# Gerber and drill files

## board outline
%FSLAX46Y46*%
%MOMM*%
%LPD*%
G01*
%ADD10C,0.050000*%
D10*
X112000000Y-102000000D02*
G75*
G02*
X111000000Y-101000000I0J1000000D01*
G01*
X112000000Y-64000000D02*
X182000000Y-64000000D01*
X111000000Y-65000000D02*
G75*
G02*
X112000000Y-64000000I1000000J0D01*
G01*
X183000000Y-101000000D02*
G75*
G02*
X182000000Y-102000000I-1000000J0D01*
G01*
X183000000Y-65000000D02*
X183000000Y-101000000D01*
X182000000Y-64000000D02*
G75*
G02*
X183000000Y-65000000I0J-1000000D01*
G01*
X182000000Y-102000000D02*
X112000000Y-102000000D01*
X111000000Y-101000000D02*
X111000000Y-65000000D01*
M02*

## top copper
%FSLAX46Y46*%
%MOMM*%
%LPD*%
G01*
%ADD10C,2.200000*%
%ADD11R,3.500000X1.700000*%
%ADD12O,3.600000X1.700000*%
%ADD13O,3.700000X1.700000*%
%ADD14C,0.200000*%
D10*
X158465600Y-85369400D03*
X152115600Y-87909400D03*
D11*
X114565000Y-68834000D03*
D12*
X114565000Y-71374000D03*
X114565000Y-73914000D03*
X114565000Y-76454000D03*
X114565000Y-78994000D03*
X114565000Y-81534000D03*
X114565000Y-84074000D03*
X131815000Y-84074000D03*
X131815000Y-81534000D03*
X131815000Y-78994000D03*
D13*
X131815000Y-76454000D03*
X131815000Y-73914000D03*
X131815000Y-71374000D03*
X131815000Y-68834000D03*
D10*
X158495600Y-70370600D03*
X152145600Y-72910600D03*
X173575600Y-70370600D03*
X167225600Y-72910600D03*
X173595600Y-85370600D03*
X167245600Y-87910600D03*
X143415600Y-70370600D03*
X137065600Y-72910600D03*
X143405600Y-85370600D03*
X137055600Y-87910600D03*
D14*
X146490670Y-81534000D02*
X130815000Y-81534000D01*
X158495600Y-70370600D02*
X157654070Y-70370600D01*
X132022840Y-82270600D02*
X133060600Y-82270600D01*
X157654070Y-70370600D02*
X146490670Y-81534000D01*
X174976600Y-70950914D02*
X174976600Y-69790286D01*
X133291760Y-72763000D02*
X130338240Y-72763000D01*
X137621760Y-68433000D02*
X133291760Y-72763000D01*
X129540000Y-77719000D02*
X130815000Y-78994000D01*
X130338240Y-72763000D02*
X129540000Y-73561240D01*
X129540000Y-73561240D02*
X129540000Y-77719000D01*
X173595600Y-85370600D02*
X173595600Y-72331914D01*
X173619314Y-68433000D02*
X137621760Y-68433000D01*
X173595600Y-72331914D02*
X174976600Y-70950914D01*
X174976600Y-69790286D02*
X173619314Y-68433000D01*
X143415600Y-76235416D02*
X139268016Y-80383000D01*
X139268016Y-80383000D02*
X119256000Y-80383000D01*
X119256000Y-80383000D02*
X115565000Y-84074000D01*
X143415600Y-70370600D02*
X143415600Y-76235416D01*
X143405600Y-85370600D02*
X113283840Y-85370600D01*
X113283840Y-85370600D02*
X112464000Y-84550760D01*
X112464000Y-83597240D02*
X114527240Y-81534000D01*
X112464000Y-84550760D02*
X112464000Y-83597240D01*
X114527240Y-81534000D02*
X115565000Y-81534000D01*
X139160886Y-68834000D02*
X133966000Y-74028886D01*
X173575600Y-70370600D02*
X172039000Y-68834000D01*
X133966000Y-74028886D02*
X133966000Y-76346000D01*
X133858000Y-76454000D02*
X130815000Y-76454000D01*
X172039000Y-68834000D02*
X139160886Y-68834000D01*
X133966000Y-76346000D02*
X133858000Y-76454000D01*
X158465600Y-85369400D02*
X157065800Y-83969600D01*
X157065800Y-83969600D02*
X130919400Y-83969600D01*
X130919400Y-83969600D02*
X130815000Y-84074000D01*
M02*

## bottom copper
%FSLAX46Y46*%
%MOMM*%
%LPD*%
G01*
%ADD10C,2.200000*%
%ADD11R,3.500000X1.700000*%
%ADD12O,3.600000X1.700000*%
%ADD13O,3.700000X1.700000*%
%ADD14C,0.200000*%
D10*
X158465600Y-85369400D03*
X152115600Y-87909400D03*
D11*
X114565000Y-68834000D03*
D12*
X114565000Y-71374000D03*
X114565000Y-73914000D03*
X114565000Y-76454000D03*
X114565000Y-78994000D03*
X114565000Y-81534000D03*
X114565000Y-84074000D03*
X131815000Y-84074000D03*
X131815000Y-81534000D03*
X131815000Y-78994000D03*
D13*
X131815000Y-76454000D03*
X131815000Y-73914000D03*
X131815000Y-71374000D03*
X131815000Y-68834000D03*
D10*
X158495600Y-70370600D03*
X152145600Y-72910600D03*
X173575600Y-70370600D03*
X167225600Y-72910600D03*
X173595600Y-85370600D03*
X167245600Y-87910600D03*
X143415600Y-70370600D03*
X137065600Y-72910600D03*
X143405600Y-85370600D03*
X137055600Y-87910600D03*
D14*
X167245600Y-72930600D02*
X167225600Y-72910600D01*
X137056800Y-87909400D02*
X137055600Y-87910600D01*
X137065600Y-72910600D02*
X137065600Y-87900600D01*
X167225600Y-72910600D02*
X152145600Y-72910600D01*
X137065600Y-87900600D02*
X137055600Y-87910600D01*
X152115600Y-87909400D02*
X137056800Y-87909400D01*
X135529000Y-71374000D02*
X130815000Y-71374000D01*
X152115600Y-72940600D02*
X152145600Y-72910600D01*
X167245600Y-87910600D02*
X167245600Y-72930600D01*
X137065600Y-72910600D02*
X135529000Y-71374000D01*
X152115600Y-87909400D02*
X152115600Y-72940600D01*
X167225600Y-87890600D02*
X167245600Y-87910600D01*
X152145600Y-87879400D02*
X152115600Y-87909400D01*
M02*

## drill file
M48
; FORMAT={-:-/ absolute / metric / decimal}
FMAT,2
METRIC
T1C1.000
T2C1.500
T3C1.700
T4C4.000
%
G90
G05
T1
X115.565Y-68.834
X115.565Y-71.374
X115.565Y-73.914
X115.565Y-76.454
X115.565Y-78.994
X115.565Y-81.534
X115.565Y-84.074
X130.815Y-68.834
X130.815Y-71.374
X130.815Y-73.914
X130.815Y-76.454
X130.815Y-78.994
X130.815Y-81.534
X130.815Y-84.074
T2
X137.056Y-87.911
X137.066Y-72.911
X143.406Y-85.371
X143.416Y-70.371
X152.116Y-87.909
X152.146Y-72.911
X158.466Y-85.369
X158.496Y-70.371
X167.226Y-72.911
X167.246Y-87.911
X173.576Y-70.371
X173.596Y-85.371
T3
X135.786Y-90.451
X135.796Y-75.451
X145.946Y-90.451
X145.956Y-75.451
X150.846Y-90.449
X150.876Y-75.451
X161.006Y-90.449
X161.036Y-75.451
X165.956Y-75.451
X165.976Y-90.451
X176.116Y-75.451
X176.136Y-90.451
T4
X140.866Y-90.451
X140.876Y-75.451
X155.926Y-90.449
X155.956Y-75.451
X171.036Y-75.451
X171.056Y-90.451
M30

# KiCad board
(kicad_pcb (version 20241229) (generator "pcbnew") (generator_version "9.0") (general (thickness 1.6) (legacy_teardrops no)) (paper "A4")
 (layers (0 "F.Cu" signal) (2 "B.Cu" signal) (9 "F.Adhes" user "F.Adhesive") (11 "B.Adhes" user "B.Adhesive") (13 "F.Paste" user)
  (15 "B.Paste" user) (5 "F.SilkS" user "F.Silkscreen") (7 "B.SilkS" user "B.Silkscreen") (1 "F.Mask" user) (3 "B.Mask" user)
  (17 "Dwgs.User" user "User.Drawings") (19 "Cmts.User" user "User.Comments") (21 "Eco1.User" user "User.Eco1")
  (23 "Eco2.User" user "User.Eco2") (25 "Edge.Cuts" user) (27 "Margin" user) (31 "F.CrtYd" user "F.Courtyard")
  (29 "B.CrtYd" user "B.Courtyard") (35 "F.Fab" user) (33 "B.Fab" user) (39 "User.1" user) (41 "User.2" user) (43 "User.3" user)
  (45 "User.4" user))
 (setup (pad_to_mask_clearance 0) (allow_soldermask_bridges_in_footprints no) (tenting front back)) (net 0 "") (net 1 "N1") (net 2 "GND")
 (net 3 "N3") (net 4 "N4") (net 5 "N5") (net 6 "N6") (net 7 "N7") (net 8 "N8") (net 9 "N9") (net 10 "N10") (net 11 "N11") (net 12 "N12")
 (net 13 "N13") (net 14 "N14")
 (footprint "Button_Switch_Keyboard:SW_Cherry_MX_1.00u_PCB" (layer "F.Cu") (at 158.4656 85.3694)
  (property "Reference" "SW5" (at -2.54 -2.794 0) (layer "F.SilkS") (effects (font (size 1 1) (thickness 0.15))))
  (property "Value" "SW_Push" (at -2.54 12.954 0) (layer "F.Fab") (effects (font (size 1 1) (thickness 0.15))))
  (pad "" np_thru_hole circle (at -7.62 5.08) (size 1.7 1.7) (drill 1.7) (layers "*.Cu" "*.Mask"))
  (pad "" np_thru_hole circle (at -2.54 5.08) (size 4 4) (drill 4) (layers "*.Cu" "*.Mask"))
  (pad "" np_thru_hole circle (at 2.54 5.08) (size 1.7 1.7) (drill 1.7) (layers "*.Cu" "*.Mask"))
  (pad "1" thru_hole circle (at 0 0) (size 2.2 2.2) (drill 1.5) (layers "*.Cu" "*.Mask") (remove_unused_layers no) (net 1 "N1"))
  (pad "2" thru_hole circle (at -6.35 2.54) (size 2.2 2.2) (drill 1.5) (layers "*.Cu" "*.Mask") (remove_unused_layers no) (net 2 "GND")))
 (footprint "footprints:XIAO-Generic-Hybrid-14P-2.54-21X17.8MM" (layer "F.Cu") (at 123.19 76.454)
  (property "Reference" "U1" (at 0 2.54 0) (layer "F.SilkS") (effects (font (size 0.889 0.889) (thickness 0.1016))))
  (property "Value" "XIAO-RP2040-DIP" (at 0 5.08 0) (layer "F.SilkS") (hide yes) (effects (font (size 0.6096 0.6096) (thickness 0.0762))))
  (pad "1" thru_hole rect (at -7.625 -7.62) (size 3.5 1.7) (drill 1 (offset -1 0)) (layers "*.Cu" "*.Mask") (remove_unused_layers no)
   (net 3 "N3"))
  (pad "2" thru_hole oval (at -7.625 -5.08) (size 3.6 1.7) (drill 1 (offset -1 0)) (layers "*.Cu" "*.Mask") (remove_unused_layers no)
   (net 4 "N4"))
  (pad "3" thru_hole oval (at -7.625 -2.54) (size 3.6 1.7) (drill 1 (offset -1 0)) (layers "*.Cu" "*.Mask") (remove_unused_layers no)
   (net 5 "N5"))
  (pad "4" thru_hole oval (at -7.625 0) (size 3.6 1.7) (drill 1 (offset -1 0)) (layers "*.Cu" "*.Mask") (remove_unused_layers no)
   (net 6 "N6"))
  (pad "5" thru_hole oval (at -7.625 2.54) (size 3.6 1.7) (drill 1 (offset -1 0)) (layers "*.Cu" "*.Mask") (remove_unused_layers no)
   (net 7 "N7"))
  (pad "6" thru_hole oval (at -7.625 5.08 180) (size 3.6 1.7) (drill 1 (offset 1 0)) (layers "*.Cu" "*.Mask") (remove_unused_layers no)
   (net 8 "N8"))
  (pad "7" thru_hole oval (at -7.625 7.62) (size 3.6 1.7) (drill 1 (offset -1 0)) (layers "*.Cu" "*.Mask") (remove_unused_layers no)
   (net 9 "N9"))
  (pad "8" thru_hole oval (at 7.625 7.62) (size 3.6 1.7) (drill 1 (offset 1 0)) (layers "*.Cu" "*.Mask") (remove_unused_layers no)
   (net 1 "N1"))
  (pad "9" thru_hole oval (at 7.625 5.08) (size 3.6 1.7) (drill 1 (offset 1 0)) (layers "*.Cu" "*.Mask") (remove_unused_layers no)
   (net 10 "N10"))
  (pad "10" thru_hole oval (at 7.625 2.54) (size 3.6 1.7) (drill 1 (offset 1 0)) (layers "*.Cu" "*.Mask") (remove_unused_layers no)
   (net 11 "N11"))
  (pad "11" thru_hole oval (at 7.625 0) (size 3.7 1.7) (drill 1 (offset 1 0)) (layers "*.Cu" "*.Mask") (remove_unused_layers no)
   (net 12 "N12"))
  (pad "12" thru_hole oval (at 7.625 -2.54) (size 3.7 1.7) (drill 1 (offset 1 0)) (layers "*.Cu" "*.Mask") (remove_unused_layers no)
   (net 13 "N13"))
  (pad "13" thru_hole oval (at 7.625 -5.08) (size 3.7 1.7) (drill 1 (offset 1 0)) (layers "*.Cu" "*.Mask") (remove_unused_layers no)
   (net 2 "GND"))
  (pad "14" thru_hole oval (at 7.625 -7.62) (size 3.7 1.7) (drill 1 (offset 1 0)) (layers "*.Cu" "*.Mask") (remove_unused_layers no)
   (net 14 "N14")))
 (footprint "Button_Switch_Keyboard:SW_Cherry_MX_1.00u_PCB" (layer "F.Cu") (at 158.4956 70.3706)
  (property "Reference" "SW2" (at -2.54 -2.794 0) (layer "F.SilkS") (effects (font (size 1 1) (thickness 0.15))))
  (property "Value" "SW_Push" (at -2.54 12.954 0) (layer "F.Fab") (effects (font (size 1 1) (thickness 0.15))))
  (pad "" np_thru_hole circle (at -7.62 5.08) (size 1.7 1.7) (drill 1.7) (layers "*.Cu" "*.Mask"))
  (pad "" np_thru_hole circle (at -2.54 5.08) (size 4 4) (drill 4) (layers "*.Cu" "*.Mask"))
  (pad "" np_thru_hole circle (at 2.54 5.08) (size 1.7 1.7) (drill 1.7) (layers "*.Cu" "*.Mask"))
  (pad "1" thru_hole circle (at 0 0) (size 2.2 2.2) (drill 1.5) (layers "*.Cu" "*.Mask") (remove_unused_layers no) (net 10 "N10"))
  (pad "2" thru_hole circle (at -6.35 2.54) (size 2.2 2.2) (drill 1.5) (layers "*.Cu" "*.Mask") (remove_unused_layers no) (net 2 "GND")))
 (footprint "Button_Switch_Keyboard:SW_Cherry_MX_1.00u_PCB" (layer "F.Cu") (at 173.5756 70.3706)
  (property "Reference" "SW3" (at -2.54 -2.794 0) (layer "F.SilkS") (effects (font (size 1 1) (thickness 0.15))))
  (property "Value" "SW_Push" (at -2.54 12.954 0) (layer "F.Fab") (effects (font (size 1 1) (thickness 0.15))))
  (pad "" np_thru_hole circle (at -7.62 5.08) (size 1.7 1.7) (drill 1.7) (layers "*.Cu" "*.Mask"))
  (pad "" np_thru_hole circle (at -2.54 5.08) (size 4 4) (drill 4) (layers "*.Cu" "*.Mask"))
  (pad "" np_thru_hole circle (at 2.54 5.08) (size 1.7 1.7) (drill 1.7) (layers "*.Cu" "*.Mask"))
  (pad "1" thru_hole circle (at 0 0) (size 2.2 2.2) (drill 1.5) (layers "*.Cu" "*.Mask") (remove_unused_layers no) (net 12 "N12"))
  (pad "2" thru_hole circle (at -6.35 2.54) (size 2.2 2.2) (drill 1.5) (layers "*.Cu" "*.Mask") (remove_unused_layers no) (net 2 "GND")))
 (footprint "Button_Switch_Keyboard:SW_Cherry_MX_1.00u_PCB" (layer "F.Cu") (at 173.5956 85.3706)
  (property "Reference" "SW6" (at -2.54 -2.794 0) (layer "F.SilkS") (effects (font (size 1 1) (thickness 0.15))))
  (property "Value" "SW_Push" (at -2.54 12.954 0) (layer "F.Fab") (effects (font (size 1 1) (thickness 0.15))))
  (pad "" np_thru_hole circle (at -7.62 5.08) (size 1.7 1.7) (drill 1.7) (layers "*.Cu" "*.Mask"))
  (pad "" np_thru_hole circle (at -2.54 5.08) (size 4 4) (drill 4) (layers "*.Cu" "*.Mask"))
  (pad "" np_thru_hole circle (at 2.54 5.08) (size 1.7 1.7) (drill 1.7) (layers "*.Cu" "*.Mask"))
  (pad "1" thru_hole circle (at 0 0) (size 2.2 2.2) (drill 1.5) (layers "*.Cu" "*.Mask") (remove_unused_layers no) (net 11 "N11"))
  (pad "2" thru_hole circle (at -6.35 2.54) (size 2.2 2.2) (drill 1.5) (layers "*.Cu" "*.Mask") (remove_unused_layers no) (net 2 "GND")))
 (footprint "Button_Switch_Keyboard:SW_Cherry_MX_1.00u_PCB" (layer "F.Cu") (at 143.4156 70.3706)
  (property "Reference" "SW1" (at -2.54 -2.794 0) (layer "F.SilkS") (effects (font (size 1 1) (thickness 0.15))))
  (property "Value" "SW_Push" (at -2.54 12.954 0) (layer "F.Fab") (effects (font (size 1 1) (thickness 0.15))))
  (pad "" np_thru_hole circle (at -7.62 5.08) (size 1.7 1.7) (drill 1.7) (layers "*.Cu" "*.Mask"))
  (pad "" np_thru_hole circle (at -2.54 5.08) (size 4 4) (drill 4) (layers "*.Cu" "*.Mask"))
  (pad "" np_thru_hole circle (at 2.54 5.08) (size 1.7 1.7) (drill 1.7) (layers "*.Cu" "*.Mask"))
  (pad "1" thru_hole circle (at 0 0) (size 2.2 2.2) (drill 1.5) (layers "*.Cu" "*.Mask") (remove_unused_layers no) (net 9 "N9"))
  (pad "2" thru_hole circle (at -6.35 2.54) (size 2.2 2.2) (drill 1.5) (layers "*.Cu" "*.Mask") (remove_unused_layers no) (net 2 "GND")))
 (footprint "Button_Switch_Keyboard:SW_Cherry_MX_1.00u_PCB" (layer "F.Cu") (at 143.4056 85.3706)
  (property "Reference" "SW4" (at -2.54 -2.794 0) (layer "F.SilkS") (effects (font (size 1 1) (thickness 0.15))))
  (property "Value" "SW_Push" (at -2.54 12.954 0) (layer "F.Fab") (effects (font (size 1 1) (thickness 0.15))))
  (pad "" np_thru_hole circle (at -7.62 5.08) (size 1.7 1.7) (drill 1.7) (layers "*.Cu" "*.Mask"))
  (pad "" np_thru_hole circle (at -2.54 5.08) (size 4 4) (drill 4) (layers "*.Cu" "*.Mask"))
  (pad "" np_thru_hole circle (at 2.54 5.08) (size 1.7 1.7) (drill 1.7) (layers "*.Cu" "*.Mask"))
  (pad "1" thru_hole circle (at 0 0) (size 2.2 2.2) (drill 1.5) (layers "*.Cu" "*.Mask") (remove_unused_layers no) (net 8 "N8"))
  (pad "2" thru_hole circle (at -6.35 2.54) (size 2.2 2.2) (drill 1.5) (layers "*.Cu" "*.Mask") (remove_unused_layers no) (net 2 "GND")))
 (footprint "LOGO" (layer "F.Cu") (at 123 94)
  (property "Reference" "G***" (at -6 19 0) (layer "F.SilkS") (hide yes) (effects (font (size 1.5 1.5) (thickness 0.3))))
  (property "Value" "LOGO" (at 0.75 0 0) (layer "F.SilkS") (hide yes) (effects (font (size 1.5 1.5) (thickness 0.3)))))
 (gr_arc (start 112 102) (mid 111.292893 101.707107) (end 111 101) (stroke (width 0.05) (type default)) (layer "Edge.Cuts"))
 (gr_line (start 112 64) (end 182 64) (stroke (width 0.05) (type default)) (layer "Edge.Cuts"))
 (gr_arc (start 111 65) (mid 111.292893 64.292893) (end 112 64) (stroke (width 0.05) (type default)) (layer "Edge.Cuts"))
 (gr_arc (start 183 101) (mid 182.707107 101.707107) (end 182 102) (stroke (width 0.05) (type default)) (layer "Edge.Cuts"))
 (gr_line (start 183 65) (end 183 101) (stroke (width 0.05) (type default)) (layer "Edge.Cuts"))
 (gr_arc (start 182 64) (mid 182.707107 64.292893) (end 183 65) (stroke (width 0.05) (type default)) (layer "Edge.Cuts"))
 (gr_line (start 182 102) (end 112 102) (stroke (width 0.05) (type default)) (layer "Edge.Cuts"))
 (gr_line (start 111 101) (end 111 65) (stroke (width 0.05) (type default)) (layer "Edge.Cuts"))
 (segment (start 146.49067 81.534) (end 130.815 81.534) (width 0.2) (layer "F.Cu") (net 10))
 (segment (start 158.4956 70.3706) (end 157.65407 70.3706) (width 0.2) (layer "F.Cu") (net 10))
 (segment (start 132.02284 82.2706) (end 133.0606 82.2706) (width 0.2) (layer "F.Cu") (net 10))
 (segment (start 157.65407 70.3706) (end 146.49067 81.534) (width 0.2) (layer "F.Cu") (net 10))
 (segment (start 167.2456 72.9306) (end 167.2256 72.9106) (width 0.2) (layer "B.Cu") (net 2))
 (segment (start 137.0568 87.9094) (end 137.0556 87.9106) (width 0.2) (layer "B.Cu") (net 2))
 (segment (start 137.0656 72.9106) (end 137.0656 87.9006) (width 0.2) (layer "B.Cu") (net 2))
 (segment (start 167.2256 72.9106) (end 152.1456 72.9106) (width 0.2) (layer "B.Cu") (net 2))
 (segment (start 137.0656 87.9006) (end 137.0556 87.9106) (width 0.2) (layer "B.Cu") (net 2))
 (segment (start 152.1156 87.9094) (end 137.0568 87.9094) (width 0.2) (layer "B.Cu") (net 2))
 (segment (start 135.529 71.374) (end 130.815 71.374) (width 0.2) (layer "B.Cu") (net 2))
 (segment (start 152.1156 72.9406) (end 152.1456 72.9106) (width 0.2) (layer "B.Cu") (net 2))
 (segment (start 167.2456 87.9106) (end 167.2456 72.9306) (width 0.2) (layer "B.Cu") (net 2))
 (segment (start 137.0656 72.9106) (end 135.529 71.374) (width 0.2) (layer "B.Cu") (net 2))
 (segment (start 152.1156 87.9094) (end 152.1156 72.9406) (width 0.2) (layer "B.Cu") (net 2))
 (segment (start 167.2256 87.8906) (end 167.2456 87.9106) (width 0.2) (layer "B.Cu") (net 2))
 (segment (start 152.1456 87.8794) (end 152.1156 87.9094) (width 0.2) (layer "B.Cu") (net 2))
 (segment (start 174.9766 70.950914) (end 174.9766 69.790286) (width 0.2) (layer "F.Cu") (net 11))
 (segment (start 133.29176 72.763) (end 130.33824 72.763) (width 0.2) (layer "F.Cu") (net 11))
 (segment (start 137.62176 68.433) (end 133.29176 72.763) (width 0.2) (layer "F.Cu") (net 11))
 (segment (start 129.54 77.719) (end 130.815 78.994) (width 0.2) (layer "F.Cu") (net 11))
 (segment (start 130.33824 72.763) (end 129.54 73.56124) (width 0.2) (layer "F.Cu") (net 11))
 (segment (start 129.54 73.56124) (end 129.54 77.719) (width 0.2) (layer "F.Cu") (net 11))
 (segment (start 173.5956 85.3706) (end 173.5956 72.331914) (width 0.2) (layer "F.Cu") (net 11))
 (segment (start 173.619314 68.433) (end 137.62176 68.433) (width 0.2) (layer "F.Cu") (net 11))
 (segment (start 173.5956 72.331914) (end 174.9766 70.950914) (width 0.2) (layer "F.Cu") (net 11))
 (segment (start 174.9766 69.790286) (end 173.619314 68.433) (width 0.2) (layer "F.Cu") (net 11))
 (segment (start 143.4156 76.235416) (end 139.268016 80.383) (width 0.2) (layer "F.Cu") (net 9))
 (segment (start 139.268016 80.383) (end 119.256 80.383) (width 0.2) (layer "F.Cu") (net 9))
 (segment (start 119.256 80.383) (end 115.565 84.074) (width 0.2) (layer "F.Cu") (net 9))
 (segment (start 143.4156 70.3706) (end 143.4156 76.235416) (width 0.2) (layer "F.Cu") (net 9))
 (segment (start 143.4056 85.3706) (end 113.28384 85.3706) (width 0.2) (layer "F.Cu") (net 8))
 (segment (start 113.28384 85.3706) (end 112.464 84.55076) (width 0.2) (layer "F.Cu") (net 8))
 (segment (start 112.464 83.59724) (end 114.52724 81.534) (width 0.2) (layer "F.Cu") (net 8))
 (segment (start 112.464 84.55076) (end 112.464 83.59724) (width 0.2) (layer "F.Cu") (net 8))
 (segment (start 114.52724 81.534) (end 115.565 81.534) (width 0.2) (layer "F.Cu") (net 8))
 (segment (start 139.160886 68.834) (end 133.966 74.028886) (width 0.2) (layer "F.Cu") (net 12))
 (segment (start 173.5756 70.3706) (end 172.039 68.834) (width 0.2) (layer "F.Cu") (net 12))
 (segment (start 133.966 74.028886) (end 133.966 76.346) (width 0.2) (layer "F.Cu") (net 12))
 (segment (start 133.858 76.454) (end 130.815 76.454) (width 0.2) (layer "F.Cu") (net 12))
 (segment (start 172.039 68.834) (end 139.160886 68.834) (width 0.2) (layer "F.Cu") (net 12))
 (segment (start 133.966 76.346) (end 133.858 76.454) (width 0.2) (layer "F.Cu") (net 12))
 (segment (start 158.4656 85.3694) (end 157.0658 83.9696) (width 0.2) (layer "F.Cu") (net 1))
 (segment (start 157.0658 83.9696) (end 130.9194 83.9696) (width 0.2) (layer "F.Cu") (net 1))
 (segment (start 130.9194 83.9696) (end 130.815 84.074) (width 0.2) (layer "F.Cu") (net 1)))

